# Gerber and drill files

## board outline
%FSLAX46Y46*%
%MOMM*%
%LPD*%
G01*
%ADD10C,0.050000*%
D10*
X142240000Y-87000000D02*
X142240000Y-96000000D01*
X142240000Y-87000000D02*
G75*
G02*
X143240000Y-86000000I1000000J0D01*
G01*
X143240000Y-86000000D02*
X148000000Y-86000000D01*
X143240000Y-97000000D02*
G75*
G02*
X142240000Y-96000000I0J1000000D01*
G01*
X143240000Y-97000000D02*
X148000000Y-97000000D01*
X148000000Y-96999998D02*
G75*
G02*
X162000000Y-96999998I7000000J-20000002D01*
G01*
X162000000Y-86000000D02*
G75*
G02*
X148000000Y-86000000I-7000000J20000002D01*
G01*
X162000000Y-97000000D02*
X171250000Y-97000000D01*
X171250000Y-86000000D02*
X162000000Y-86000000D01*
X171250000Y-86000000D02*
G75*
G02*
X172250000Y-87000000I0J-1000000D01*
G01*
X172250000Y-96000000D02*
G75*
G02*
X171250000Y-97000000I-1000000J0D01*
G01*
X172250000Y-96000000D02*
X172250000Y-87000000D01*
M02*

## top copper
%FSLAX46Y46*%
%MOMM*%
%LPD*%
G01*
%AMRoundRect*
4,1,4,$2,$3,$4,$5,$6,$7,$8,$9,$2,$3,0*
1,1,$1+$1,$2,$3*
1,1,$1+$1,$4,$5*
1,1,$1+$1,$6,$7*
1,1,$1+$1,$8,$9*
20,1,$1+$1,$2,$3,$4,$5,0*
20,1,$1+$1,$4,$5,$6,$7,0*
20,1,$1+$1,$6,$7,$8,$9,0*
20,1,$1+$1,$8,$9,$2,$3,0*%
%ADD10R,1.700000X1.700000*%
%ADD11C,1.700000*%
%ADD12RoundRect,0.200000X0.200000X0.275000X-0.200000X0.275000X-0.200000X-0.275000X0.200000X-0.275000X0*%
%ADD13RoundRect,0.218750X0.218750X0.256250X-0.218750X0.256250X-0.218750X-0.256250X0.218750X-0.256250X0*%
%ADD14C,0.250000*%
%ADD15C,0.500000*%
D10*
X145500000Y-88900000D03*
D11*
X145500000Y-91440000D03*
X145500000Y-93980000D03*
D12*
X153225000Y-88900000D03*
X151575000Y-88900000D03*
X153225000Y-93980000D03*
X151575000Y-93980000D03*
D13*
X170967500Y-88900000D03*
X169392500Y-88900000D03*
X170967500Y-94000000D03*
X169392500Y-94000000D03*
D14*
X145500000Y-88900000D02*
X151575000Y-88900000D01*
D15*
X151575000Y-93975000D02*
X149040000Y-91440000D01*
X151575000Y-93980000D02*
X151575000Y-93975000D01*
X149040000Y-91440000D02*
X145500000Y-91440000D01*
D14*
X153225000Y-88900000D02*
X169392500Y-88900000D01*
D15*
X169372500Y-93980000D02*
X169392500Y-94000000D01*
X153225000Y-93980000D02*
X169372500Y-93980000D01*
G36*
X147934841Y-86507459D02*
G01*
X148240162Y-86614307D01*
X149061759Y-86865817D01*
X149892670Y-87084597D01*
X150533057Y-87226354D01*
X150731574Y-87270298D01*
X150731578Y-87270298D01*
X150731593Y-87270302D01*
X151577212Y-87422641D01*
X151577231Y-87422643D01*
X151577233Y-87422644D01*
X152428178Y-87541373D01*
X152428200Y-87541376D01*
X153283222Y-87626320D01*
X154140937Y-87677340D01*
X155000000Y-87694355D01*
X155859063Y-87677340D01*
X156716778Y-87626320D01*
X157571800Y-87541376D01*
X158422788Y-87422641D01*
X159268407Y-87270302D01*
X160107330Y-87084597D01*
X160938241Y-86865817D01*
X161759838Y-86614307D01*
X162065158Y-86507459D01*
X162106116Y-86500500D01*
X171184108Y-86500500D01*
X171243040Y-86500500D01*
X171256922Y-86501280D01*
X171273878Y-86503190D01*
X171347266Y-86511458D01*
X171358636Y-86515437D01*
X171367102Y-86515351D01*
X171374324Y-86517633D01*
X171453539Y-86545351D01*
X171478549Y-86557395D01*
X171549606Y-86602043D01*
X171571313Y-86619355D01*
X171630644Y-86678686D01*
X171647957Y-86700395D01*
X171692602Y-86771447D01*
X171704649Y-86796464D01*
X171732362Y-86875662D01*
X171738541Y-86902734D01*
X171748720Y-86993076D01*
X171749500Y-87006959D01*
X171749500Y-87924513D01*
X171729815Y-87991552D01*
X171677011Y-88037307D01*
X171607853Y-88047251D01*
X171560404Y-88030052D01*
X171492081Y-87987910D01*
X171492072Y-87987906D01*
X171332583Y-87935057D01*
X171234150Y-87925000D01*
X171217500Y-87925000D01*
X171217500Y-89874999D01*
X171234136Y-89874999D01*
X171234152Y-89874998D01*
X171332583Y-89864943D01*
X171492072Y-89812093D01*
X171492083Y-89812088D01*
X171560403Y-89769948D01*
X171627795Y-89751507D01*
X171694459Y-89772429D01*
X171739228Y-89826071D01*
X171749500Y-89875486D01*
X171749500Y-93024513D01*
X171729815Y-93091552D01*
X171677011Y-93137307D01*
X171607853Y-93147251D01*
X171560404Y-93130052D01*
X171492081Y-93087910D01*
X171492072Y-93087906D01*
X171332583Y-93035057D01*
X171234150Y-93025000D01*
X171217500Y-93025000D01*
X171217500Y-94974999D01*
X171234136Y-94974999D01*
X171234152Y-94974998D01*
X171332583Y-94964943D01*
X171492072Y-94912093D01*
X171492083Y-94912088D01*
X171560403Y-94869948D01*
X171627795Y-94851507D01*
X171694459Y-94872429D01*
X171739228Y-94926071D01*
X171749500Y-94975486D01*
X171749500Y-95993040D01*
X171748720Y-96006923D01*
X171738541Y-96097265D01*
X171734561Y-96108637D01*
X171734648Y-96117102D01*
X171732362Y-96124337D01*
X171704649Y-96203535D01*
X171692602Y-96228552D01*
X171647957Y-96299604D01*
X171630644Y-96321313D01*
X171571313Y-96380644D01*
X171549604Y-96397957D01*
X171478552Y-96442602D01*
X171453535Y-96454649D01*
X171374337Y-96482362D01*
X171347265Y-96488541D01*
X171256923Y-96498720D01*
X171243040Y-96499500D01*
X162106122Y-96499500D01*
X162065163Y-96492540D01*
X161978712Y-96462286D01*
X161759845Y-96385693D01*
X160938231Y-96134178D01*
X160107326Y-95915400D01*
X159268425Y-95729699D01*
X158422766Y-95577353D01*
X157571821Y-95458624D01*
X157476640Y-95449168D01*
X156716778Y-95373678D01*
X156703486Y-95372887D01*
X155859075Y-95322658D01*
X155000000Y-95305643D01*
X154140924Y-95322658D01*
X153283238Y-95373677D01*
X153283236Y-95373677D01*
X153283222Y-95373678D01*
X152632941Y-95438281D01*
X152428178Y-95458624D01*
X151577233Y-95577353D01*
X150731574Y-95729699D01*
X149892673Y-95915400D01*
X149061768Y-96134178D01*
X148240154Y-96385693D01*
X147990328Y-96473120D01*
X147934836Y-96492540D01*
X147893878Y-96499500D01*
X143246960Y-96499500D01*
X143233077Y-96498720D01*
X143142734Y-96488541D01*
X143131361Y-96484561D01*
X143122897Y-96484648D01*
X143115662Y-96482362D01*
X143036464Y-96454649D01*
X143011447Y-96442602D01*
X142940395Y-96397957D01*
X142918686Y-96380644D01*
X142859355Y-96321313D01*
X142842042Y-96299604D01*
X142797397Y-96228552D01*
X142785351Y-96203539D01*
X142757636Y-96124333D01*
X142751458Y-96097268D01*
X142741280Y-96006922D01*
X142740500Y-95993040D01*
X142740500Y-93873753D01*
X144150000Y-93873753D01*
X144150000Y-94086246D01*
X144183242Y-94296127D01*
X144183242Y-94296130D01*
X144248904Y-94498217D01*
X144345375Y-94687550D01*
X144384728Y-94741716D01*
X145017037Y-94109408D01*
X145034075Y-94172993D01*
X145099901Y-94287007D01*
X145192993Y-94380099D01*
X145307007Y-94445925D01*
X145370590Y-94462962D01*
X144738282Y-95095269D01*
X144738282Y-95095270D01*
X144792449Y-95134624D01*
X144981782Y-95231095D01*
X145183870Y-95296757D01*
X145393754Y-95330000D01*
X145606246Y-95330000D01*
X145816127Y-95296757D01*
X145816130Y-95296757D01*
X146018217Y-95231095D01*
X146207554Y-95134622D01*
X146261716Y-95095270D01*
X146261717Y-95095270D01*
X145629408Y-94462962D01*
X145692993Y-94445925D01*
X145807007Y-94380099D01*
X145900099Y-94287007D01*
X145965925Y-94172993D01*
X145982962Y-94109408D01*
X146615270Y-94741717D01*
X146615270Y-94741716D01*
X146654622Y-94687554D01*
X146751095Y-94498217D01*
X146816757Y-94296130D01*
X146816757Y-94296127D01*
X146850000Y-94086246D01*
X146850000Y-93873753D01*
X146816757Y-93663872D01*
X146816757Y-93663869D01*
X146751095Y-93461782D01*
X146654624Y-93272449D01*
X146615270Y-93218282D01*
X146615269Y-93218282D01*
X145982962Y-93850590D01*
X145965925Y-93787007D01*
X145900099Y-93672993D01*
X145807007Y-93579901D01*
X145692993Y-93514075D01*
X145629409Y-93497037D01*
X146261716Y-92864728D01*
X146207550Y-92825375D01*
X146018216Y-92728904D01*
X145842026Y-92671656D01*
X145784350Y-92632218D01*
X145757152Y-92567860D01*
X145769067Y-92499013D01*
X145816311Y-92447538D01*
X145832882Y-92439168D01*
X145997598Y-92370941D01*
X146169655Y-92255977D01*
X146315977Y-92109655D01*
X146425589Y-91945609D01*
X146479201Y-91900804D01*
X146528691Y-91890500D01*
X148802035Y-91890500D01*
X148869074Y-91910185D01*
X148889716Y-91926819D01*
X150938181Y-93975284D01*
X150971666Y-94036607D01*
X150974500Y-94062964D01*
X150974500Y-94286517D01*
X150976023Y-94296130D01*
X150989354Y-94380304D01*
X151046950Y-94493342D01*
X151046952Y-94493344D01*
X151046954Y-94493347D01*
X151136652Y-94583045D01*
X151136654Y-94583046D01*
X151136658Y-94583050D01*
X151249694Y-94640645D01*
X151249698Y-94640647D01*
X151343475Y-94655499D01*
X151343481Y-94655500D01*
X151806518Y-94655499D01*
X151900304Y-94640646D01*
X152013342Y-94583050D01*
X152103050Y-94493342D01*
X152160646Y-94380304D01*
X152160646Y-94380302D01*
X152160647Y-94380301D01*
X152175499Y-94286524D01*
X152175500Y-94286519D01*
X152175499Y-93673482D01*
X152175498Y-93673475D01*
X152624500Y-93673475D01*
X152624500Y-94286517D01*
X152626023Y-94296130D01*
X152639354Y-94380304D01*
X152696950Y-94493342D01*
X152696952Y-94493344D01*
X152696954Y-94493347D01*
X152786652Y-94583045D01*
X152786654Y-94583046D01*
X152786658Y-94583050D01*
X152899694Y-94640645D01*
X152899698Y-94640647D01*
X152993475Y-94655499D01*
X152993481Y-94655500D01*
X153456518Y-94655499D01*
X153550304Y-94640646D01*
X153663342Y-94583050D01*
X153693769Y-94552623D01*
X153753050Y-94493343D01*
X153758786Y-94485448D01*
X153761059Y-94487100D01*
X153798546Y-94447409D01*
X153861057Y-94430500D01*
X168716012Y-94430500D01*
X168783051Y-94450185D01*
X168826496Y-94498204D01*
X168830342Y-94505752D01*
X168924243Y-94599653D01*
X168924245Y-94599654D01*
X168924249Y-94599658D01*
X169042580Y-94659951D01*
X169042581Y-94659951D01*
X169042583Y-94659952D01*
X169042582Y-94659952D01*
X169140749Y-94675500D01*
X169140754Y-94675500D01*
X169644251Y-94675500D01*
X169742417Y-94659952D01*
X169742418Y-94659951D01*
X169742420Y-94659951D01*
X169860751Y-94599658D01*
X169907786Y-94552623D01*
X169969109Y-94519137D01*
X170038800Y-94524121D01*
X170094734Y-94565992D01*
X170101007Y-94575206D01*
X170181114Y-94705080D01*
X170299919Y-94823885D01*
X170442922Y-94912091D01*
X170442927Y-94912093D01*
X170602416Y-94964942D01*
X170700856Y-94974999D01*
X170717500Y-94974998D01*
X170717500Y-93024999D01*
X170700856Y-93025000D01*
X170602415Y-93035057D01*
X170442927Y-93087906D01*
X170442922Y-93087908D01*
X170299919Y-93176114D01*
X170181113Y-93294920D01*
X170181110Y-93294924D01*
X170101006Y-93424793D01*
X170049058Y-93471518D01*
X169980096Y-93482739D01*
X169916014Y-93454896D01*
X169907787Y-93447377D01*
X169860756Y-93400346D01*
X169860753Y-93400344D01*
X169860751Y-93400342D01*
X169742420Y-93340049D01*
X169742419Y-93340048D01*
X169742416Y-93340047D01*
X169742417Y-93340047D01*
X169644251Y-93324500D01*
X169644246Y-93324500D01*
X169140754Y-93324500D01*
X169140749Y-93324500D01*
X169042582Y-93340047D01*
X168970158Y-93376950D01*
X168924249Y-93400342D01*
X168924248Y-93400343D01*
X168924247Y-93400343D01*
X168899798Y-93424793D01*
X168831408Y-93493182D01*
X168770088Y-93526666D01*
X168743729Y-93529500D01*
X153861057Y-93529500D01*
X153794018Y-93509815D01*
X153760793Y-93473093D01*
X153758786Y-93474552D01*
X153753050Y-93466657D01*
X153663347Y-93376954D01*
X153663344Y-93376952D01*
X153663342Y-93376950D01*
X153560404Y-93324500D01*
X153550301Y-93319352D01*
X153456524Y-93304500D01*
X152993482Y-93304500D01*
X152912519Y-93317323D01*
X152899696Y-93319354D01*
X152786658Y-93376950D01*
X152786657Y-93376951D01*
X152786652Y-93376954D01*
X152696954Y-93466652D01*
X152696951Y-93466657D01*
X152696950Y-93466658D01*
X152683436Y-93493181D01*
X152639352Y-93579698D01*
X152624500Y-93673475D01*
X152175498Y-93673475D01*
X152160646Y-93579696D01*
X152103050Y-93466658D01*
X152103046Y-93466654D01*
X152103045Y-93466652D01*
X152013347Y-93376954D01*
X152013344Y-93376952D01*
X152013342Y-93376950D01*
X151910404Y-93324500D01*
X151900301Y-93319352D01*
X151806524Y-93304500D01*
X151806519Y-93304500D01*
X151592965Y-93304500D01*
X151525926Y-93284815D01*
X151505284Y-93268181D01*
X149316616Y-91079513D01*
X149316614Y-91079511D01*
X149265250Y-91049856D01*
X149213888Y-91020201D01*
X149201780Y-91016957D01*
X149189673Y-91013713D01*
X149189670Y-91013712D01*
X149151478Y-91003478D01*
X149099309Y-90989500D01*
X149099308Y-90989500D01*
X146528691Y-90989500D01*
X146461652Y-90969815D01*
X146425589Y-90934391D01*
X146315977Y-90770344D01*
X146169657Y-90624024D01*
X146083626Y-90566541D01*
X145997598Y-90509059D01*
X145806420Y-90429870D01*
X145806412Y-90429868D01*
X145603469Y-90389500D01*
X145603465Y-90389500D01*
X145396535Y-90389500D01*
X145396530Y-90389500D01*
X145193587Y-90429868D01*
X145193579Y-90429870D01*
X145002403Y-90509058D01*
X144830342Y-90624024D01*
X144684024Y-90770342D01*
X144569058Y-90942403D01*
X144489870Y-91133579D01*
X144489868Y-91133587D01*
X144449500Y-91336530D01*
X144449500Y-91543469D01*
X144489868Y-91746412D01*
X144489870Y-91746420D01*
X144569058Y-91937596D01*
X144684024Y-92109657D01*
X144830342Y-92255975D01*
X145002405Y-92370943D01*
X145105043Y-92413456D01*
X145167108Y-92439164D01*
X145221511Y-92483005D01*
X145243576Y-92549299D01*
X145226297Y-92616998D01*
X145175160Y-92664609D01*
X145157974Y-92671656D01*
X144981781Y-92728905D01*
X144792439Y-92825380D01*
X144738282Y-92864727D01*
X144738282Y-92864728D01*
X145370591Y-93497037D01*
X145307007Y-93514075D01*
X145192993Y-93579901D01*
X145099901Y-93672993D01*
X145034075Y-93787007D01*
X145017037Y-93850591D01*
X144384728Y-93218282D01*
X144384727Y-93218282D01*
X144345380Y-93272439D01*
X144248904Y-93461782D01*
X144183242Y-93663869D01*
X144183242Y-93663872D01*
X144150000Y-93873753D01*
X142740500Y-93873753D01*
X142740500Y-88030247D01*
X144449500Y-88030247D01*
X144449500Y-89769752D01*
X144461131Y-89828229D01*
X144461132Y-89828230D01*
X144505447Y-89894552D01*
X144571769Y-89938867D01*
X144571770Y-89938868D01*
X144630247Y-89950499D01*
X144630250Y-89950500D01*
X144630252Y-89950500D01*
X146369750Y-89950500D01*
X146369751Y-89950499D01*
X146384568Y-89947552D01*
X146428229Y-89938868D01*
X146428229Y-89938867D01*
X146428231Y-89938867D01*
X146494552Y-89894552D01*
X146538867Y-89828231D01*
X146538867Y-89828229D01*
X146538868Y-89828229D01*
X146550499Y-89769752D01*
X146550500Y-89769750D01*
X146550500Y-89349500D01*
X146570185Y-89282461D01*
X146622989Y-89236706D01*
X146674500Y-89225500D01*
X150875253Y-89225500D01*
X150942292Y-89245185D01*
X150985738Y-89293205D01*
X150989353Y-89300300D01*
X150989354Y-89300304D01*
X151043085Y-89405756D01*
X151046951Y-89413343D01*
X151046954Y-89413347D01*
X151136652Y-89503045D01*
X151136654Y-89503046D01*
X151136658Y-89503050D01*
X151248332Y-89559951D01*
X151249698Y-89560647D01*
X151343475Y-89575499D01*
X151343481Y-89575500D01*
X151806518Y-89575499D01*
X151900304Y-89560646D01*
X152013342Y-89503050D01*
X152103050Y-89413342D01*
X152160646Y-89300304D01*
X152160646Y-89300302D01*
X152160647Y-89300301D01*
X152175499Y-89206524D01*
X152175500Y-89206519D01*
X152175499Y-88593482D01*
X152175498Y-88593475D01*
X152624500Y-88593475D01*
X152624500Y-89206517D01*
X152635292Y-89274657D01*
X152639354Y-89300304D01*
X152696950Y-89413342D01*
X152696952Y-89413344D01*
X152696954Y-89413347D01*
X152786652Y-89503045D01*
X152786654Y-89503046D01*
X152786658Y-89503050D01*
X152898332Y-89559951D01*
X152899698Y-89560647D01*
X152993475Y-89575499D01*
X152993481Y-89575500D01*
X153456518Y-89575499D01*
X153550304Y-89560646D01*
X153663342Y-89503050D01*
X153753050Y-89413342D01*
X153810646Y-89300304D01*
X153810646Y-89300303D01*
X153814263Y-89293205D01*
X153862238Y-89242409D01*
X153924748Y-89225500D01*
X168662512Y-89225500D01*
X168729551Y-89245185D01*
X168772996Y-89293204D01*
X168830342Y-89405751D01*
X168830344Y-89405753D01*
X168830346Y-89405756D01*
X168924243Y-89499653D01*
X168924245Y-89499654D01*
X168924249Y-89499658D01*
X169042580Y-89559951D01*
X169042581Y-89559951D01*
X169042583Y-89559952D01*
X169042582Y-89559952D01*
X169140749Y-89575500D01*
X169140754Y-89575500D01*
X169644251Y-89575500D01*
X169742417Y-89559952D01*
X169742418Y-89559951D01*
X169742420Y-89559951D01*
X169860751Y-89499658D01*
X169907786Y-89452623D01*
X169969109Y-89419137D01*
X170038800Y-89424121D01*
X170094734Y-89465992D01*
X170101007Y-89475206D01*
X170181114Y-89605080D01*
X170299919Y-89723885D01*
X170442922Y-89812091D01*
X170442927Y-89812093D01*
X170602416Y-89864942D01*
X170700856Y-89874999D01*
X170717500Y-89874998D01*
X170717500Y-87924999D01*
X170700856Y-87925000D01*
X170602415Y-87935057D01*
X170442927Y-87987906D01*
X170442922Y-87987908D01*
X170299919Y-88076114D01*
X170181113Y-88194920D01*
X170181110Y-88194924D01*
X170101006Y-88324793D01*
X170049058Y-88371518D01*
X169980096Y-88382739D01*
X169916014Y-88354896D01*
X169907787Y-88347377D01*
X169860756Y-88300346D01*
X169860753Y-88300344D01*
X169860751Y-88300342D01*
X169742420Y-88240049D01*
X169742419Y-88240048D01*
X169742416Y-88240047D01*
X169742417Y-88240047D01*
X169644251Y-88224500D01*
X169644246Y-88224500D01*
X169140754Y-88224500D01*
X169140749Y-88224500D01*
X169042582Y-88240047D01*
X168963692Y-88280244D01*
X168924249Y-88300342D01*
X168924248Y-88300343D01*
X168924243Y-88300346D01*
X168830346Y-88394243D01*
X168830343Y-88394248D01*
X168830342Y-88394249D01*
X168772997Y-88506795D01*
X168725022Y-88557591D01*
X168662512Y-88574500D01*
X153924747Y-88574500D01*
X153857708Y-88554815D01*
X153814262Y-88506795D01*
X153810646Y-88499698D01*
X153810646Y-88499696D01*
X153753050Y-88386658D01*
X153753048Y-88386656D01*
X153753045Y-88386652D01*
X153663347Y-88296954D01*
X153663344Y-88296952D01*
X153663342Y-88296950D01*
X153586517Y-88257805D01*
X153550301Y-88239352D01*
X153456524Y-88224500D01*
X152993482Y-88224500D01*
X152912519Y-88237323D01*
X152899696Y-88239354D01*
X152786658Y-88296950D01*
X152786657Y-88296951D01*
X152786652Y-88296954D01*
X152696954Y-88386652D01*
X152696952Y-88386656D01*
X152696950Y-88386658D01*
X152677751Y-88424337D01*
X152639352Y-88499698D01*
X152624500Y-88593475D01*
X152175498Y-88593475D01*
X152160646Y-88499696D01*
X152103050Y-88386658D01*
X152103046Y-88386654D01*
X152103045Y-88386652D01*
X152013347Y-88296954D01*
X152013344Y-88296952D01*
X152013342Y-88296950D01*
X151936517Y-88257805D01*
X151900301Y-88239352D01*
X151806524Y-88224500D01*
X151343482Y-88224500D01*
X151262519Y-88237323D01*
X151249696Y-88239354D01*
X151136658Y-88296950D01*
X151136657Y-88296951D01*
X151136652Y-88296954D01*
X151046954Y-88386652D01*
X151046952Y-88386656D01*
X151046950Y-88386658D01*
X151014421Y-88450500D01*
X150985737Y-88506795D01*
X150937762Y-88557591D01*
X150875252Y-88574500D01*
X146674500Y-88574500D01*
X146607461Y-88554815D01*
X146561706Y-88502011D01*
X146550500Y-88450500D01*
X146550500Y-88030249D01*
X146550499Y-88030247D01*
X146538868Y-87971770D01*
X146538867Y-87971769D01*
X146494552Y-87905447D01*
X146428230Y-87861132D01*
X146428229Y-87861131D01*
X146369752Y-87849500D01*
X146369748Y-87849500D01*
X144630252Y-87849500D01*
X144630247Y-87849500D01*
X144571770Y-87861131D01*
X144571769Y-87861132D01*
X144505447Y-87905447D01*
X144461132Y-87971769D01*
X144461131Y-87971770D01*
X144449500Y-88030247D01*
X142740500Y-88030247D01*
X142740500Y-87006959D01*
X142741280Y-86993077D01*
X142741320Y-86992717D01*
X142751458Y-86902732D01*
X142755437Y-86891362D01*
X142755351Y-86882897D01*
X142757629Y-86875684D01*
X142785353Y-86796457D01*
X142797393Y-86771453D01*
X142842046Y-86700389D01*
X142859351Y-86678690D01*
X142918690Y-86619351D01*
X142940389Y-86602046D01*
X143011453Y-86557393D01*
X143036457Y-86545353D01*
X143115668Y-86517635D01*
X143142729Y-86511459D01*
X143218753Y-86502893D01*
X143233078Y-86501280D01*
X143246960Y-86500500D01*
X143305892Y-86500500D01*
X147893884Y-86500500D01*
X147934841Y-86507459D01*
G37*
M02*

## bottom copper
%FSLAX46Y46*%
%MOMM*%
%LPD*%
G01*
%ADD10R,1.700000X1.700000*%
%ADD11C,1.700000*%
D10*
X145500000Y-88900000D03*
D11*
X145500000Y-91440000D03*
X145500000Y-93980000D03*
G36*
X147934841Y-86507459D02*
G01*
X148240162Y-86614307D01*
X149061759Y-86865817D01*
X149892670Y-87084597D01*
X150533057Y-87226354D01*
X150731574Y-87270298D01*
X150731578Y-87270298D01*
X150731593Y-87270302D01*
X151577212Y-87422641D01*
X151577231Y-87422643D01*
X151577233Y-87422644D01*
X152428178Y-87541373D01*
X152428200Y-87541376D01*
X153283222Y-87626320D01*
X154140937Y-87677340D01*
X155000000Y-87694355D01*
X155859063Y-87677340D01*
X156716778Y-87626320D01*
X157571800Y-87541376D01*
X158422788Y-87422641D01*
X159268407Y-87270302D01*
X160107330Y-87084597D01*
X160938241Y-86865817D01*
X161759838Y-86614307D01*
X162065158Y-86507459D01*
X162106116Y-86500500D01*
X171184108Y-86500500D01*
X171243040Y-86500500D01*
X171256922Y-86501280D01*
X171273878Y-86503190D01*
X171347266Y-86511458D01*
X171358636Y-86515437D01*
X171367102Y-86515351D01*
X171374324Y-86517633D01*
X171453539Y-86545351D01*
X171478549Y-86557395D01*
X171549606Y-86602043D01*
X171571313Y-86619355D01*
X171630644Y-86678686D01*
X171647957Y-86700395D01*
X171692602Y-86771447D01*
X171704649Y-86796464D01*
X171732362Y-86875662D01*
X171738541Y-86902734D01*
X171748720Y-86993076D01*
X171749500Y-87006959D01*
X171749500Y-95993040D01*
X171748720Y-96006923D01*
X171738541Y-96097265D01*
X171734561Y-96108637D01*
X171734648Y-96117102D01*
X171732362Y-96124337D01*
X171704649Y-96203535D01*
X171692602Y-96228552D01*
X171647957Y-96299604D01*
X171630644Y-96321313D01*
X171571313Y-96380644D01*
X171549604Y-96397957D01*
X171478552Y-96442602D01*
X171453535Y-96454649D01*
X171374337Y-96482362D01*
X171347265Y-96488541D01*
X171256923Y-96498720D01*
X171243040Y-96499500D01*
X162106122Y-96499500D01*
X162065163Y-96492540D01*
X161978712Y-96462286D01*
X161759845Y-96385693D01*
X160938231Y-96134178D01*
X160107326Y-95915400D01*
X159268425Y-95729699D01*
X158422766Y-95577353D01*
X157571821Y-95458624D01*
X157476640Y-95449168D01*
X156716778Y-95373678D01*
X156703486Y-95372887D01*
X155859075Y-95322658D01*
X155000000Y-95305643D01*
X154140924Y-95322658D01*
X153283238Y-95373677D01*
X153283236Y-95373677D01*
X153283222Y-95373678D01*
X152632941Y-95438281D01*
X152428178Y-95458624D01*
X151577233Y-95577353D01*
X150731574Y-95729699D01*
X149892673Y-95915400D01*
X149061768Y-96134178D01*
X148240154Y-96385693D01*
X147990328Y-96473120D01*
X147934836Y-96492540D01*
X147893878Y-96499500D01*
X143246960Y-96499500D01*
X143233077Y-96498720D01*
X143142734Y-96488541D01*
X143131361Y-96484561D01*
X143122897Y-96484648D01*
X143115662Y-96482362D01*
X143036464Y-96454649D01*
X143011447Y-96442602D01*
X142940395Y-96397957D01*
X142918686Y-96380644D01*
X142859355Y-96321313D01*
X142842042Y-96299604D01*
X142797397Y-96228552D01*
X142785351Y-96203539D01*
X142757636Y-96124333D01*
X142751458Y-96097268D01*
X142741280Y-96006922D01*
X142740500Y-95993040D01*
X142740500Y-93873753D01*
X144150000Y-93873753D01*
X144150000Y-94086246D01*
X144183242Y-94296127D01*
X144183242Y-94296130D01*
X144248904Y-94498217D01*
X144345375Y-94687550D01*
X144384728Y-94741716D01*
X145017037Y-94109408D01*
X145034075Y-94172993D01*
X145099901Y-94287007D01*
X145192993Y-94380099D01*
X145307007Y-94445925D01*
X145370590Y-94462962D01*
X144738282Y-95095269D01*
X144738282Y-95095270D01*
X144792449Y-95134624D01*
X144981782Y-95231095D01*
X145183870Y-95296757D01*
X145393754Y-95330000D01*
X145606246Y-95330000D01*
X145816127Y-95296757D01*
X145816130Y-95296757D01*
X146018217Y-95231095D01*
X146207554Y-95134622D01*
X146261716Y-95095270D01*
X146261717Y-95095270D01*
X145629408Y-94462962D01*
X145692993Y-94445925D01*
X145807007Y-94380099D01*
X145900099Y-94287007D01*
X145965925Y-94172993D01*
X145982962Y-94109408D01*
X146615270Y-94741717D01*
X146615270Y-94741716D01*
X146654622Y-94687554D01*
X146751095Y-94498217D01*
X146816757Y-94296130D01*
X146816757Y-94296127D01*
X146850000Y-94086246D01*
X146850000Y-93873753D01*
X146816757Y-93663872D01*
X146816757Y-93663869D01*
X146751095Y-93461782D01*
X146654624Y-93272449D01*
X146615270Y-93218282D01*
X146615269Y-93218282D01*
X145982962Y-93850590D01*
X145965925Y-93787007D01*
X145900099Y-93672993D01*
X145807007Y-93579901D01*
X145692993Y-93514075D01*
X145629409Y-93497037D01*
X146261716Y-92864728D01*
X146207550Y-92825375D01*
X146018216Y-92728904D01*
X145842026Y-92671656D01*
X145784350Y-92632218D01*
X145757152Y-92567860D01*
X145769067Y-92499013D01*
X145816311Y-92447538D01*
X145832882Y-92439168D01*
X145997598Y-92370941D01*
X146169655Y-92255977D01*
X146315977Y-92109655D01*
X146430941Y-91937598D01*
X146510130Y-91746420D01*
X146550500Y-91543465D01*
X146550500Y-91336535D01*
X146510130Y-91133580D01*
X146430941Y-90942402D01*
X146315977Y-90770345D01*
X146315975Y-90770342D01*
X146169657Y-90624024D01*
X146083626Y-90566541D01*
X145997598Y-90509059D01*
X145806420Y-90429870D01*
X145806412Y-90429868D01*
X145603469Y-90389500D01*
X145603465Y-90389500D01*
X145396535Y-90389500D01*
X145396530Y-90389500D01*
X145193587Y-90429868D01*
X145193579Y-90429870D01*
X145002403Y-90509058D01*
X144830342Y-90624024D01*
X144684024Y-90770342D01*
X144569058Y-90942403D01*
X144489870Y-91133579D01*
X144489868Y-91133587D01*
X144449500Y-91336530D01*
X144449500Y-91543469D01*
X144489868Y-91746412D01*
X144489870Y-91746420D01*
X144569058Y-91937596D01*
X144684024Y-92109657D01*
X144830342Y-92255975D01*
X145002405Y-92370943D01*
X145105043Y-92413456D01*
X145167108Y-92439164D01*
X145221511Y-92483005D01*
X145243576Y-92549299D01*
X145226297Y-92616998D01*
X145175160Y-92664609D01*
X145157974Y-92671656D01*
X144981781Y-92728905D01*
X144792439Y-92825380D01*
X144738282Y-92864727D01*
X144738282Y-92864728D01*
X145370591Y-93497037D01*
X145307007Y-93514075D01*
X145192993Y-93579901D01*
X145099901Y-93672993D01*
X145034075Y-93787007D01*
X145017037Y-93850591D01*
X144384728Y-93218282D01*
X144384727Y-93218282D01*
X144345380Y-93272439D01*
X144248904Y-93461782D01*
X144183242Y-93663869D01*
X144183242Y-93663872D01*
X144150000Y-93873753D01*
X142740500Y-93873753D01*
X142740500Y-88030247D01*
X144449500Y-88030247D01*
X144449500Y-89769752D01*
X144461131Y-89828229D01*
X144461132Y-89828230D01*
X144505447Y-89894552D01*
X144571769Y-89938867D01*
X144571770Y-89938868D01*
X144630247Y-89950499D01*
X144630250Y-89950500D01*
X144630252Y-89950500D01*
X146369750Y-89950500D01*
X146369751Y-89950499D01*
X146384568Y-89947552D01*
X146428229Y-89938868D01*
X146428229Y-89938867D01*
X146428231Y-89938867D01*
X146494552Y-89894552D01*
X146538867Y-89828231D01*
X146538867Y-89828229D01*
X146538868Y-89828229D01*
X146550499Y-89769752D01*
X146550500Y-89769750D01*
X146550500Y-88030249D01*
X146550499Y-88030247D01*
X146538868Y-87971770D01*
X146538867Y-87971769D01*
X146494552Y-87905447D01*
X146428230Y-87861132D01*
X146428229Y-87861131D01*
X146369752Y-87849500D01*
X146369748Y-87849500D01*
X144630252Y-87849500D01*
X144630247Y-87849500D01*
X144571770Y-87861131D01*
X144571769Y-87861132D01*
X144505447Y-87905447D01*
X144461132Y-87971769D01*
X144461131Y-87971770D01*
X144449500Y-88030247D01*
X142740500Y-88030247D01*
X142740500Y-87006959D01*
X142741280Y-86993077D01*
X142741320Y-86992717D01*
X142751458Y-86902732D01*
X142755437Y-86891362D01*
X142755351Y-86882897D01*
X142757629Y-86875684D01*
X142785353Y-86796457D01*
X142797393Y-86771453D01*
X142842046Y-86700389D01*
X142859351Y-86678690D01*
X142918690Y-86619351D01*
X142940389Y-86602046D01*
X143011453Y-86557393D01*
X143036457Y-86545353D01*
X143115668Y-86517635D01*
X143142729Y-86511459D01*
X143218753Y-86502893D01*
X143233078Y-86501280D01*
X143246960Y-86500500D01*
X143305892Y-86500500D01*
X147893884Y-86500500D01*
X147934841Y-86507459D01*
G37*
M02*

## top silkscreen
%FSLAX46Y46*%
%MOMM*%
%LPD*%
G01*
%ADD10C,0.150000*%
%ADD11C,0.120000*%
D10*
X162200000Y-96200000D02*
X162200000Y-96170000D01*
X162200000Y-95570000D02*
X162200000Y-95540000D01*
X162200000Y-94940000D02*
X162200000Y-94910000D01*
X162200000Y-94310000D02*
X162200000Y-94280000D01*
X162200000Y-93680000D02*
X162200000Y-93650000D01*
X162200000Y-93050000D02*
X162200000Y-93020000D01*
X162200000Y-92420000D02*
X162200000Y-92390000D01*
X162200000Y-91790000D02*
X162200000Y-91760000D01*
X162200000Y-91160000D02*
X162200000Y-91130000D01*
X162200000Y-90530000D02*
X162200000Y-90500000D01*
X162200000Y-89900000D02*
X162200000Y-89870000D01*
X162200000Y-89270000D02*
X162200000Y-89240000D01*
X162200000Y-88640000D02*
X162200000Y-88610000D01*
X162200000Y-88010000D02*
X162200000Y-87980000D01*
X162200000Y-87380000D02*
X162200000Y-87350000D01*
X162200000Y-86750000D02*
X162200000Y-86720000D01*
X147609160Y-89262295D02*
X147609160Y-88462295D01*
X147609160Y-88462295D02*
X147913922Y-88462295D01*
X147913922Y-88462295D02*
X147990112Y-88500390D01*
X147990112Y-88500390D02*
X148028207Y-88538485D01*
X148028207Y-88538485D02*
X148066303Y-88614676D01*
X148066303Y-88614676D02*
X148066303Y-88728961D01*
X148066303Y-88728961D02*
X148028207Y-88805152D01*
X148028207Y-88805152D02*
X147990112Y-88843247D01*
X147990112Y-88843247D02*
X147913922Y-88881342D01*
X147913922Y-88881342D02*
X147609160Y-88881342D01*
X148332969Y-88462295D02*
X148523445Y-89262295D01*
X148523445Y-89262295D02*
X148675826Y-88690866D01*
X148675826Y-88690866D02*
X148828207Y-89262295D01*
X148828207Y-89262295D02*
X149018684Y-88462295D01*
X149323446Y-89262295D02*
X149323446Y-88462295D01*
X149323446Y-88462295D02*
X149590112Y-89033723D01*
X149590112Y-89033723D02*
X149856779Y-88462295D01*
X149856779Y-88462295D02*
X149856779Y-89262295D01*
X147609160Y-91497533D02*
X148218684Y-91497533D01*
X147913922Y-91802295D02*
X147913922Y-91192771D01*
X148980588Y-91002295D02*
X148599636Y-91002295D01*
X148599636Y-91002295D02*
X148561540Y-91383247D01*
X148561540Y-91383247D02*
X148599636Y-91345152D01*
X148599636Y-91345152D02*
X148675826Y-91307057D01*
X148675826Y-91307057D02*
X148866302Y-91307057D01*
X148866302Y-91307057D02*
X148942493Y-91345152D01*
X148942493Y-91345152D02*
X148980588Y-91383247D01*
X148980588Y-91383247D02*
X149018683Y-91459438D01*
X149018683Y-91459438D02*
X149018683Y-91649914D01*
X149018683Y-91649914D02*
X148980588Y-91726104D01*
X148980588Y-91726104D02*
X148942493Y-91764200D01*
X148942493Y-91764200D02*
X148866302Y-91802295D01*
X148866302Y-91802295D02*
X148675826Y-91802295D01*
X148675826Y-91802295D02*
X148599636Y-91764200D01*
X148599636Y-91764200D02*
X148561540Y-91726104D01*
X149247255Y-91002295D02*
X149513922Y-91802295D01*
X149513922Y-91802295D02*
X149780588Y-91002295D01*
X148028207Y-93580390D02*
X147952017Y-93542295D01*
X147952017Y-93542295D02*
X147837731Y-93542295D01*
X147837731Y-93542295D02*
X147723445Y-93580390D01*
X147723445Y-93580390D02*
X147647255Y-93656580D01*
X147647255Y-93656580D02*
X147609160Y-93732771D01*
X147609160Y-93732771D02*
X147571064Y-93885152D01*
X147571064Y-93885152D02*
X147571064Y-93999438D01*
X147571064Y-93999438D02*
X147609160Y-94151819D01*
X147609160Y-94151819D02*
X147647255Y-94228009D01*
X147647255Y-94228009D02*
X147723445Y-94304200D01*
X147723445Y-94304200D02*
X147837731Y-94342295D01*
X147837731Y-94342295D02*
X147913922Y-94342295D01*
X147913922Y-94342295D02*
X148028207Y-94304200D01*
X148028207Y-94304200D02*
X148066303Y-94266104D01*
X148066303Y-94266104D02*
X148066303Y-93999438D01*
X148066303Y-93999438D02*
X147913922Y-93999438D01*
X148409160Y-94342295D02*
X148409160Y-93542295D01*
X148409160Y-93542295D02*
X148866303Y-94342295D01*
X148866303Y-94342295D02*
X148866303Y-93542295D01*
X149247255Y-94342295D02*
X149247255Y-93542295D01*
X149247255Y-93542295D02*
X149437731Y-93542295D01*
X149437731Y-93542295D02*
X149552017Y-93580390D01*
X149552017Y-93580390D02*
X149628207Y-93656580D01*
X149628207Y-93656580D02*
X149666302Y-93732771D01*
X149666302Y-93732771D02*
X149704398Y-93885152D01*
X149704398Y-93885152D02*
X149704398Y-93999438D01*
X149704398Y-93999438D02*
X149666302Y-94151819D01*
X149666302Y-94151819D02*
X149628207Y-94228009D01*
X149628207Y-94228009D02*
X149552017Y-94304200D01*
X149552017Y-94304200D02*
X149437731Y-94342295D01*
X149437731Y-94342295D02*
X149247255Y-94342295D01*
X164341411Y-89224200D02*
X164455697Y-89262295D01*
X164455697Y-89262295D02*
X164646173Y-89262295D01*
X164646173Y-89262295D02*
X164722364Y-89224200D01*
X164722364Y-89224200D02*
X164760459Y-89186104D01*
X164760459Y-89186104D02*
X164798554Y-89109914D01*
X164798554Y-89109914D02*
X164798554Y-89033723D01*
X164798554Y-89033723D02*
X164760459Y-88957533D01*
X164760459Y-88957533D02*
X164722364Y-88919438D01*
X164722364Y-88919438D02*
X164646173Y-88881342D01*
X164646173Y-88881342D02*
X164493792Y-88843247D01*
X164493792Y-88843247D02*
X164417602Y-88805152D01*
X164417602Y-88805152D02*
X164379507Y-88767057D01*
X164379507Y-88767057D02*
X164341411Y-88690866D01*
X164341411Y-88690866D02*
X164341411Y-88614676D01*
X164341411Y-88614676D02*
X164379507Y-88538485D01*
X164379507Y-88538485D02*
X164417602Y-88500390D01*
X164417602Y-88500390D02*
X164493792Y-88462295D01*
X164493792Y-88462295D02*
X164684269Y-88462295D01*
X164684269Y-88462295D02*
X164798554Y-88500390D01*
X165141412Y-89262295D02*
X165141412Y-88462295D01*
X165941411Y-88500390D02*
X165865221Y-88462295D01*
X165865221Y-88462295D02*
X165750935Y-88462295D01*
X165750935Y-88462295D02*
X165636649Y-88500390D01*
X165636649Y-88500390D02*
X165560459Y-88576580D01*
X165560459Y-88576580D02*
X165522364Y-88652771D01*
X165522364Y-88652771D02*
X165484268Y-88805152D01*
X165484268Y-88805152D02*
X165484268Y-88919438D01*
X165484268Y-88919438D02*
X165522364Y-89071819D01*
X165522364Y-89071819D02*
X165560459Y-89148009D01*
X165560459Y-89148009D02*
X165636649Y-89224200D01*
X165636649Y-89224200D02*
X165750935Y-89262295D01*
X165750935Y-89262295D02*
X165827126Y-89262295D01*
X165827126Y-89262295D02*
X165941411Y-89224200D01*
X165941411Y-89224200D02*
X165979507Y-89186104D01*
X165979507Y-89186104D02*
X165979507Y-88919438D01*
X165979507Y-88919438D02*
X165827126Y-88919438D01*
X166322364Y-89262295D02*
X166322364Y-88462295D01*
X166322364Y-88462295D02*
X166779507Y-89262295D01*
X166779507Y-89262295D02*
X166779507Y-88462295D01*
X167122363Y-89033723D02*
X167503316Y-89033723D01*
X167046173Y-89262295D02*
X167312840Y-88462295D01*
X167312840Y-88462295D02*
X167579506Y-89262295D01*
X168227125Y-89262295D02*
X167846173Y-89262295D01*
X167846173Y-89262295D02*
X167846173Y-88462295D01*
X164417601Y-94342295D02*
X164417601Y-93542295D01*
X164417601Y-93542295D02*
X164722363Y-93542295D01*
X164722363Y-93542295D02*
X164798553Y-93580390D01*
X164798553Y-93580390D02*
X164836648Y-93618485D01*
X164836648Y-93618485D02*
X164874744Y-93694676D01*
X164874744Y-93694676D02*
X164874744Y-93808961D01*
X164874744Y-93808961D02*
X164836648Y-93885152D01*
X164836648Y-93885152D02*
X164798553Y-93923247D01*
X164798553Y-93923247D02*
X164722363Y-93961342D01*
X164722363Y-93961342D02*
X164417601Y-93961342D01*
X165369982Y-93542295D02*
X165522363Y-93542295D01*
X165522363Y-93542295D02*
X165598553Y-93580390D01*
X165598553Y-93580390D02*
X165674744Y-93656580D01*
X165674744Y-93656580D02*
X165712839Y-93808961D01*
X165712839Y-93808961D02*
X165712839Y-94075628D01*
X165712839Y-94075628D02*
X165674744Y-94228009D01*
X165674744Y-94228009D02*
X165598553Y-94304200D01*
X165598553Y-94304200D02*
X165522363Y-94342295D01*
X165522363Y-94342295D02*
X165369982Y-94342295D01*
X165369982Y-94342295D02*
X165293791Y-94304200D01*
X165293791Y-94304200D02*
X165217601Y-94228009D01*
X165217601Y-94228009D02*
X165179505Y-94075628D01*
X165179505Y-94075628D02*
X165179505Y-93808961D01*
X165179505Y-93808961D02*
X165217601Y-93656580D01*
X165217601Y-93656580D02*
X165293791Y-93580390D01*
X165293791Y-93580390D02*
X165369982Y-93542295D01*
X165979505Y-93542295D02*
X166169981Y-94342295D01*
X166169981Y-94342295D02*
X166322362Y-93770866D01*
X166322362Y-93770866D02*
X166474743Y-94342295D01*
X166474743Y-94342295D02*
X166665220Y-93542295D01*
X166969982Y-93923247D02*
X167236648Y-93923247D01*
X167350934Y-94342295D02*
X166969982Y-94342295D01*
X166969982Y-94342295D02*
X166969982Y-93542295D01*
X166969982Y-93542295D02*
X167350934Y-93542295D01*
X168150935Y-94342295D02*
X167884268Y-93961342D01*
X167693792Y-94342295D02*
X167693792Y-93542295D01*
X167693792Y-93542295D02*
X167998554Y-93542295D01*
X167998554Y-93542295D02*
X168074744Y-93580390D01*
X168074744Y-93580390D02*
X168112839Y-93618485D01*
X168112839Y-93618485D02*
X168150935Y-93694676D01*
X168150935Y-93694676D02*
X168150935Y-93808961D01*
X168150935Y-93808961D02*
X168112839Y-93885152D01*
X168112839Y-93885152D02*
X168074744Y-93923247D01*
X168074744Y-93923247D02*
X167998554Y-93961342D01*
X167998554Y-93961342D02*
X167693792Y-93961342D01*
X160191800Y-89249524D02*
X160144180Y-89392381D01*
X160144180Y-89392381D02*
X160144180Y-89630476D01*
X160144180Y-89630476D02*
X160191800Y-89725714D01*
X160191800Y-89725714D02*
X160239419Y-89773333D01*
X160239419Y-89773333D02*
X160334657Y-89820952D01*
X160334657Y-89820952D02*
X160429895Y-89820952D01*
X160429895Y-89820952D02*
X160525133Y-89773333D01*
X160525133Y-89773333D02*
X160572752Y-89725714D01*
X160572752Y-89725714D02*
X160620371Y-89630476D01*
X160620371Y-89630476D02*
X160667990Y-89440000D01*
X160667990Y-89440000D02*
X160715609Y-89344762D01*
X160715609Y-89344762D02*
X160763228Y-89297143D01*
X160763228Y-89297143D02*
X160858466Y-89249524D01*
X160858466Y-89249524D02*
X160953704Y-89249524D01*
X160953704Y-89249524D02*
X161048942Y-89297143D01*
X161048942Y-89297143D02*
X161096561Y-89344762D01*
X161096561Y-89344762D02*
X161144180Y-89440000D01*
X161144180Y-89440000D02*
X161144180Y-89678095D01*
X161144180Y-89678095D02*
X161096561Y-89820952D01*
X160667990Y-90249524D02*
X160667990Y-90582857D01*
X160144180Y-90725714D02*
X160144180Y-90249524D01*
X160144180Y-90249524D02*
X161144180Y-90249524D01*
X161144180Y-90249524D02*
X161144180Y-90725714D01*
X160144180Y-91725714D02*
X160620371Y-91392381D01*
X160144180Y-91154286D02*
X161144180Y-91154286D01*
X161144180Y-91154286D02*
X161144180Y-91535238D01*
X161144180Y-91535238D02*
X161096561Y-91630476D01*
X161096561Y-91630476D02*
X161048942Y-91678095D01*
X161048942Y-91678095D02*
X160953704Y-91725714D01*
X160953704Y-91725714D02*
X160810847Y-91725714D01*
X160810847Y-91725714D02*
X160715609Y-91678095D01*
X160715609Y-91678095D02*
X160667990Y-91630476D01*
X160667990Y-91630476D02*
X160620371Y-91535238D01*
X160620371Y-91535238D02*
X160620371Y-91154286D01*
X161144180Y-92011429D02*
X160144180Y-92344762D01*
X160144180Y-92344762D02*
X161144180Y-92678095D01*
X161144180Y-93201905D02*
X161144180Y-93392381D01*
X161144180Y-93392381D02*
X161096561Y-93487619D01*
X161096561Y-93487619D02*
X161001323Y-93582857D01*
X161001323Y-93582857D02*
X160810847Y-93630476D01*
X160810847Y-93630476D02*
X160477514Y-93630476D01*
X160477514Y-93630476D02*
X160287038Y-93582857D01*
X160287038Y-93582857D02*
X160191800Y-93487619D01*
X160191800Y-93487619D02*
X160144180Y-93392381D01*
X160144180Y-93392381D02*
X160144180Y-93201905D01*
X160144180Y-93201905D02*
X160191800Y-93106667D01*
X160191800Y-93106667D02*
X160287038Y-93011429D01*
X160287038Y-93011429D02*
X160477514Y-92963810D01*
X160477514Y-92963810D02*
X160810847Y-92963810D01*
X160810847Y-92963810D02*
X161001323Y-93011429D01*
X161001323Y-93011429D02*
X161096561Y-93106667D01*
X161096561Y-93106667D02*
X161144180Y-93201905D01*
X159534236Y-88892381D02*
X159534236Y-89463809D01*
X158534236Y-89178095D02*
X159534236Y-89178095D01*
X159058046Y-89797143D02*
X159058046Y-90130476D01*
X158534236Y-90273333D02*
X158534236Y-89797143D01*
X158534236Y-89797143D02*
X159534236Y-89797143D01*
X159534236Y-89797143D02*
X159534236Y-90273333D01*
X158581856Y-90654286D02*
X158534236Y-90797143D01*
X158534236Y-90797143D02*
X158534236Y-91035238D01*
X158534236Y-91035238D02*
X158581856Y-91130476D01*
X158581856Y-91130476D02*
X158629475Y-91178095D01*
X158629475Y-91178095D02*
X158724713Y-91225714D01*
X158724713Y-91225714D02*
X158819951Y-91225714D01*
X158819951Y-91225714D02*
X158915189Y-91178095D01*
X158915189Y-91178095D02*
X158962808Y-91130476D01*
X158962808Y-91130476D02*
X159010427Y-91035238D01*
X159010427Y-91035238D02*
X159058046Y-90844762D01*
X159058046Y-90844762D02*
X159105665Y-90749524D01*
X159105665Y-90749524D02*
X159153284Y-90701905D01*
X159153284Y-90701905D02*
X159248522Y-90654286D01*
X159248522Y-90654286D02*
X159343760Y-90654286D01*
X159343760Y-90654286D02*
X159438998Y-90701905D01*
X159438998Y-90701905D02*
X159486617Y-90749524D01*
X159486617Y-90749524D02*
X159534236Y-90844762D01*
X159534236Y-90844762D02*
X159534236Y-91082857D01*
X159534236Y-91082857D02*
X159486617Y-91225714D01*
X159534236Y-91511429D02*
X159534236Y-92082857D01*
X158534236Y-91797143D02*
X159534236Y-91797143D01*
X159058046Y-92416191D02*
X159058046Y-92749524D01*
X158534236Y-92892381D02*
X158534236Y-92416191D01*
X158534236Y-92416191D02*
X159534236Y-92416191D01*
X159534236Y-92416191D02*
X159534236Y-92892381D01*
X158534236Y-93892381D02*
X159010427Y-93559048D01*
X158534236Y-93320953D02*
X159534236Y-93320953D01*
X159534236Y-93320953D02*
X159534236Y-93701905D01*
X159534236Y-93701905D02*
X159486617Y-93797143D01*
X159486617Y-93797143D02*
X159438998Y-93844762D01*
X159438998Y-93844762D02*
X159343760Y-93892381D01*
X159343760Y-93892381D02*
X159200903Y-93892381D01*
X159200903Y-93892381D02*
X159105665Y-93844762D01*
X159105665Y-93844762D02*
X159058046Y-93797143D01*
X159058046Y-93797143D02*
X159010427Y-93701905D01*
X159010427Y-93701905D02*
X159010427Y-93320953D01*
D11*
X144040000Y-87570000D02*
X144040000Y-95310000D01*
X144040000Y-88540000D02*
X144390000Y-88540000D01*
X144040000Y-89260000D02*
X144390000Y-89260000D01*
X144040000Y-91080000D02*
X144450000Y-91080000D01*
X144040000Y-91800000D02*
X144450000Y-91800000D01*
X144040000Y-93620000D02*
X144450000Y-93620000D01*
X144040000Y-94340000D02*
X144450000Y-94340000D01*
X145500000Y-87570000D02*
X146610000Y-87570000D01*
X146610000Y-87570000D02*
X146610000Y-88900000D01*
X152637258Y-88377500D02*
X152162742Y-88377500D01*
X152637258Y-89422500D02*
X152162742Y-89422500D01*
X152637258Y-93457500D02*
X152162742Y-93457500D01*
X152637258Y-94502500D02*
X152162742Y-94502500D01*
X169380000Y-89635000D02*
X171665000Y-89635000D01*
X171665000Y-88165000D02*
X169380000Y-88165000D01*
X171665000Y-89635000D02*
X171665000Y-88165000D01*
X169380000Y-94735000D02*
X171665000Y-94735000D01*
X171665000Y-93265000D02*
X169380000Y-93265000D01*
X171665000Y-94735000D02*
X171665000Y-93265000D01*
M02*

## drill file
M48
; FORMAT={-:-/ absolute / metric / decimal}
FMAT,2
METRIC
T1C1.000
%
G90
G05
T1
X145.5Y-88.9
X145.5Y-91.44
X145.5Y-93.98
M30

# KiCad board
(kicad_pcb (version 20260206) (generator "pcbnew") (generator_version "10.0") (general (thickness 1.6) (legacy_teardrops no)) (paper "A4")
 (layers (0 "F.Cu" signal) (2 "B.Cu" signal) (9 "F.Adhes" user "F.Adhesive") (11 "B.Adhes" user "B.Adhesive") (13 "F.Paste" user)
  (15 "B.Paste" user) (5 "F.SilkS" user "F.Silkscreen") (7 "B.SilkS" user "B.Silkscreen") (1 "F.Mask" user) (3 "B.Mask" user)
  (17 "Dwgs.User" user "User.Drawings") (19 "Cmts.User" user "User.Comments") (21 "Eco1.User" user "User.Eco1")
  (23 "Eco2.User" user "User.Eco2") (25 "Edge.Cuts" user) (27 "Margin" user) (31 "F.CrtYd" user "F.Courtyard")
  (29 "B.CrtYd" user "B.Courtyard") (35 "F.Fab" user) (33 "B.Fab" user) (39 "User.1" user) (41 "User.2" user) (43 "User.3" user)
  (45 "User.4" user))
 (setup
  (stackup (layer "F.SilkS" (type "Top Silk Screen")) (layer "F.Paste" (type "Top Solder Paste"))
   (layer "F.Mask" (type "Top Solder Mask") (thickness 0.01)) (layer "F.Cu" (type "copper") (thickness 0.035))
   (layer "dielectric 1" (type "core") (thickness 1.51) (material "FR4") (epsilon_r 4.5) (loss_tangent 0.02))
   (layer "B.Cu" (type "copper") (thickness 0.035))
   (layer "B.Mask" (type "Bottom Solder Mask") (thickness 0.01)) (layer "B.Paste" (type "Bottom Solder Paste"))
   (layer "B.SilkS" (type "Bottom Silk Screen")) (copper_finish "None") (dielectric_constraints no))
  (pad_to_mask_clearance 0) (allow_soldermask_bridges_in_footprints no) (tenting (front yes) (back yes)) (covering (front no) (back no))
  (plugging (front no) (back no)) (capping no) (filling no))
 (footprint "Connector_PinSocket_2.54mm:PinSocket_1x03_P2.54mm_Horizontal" (layer "F.Cu") (at 145.5 88.9)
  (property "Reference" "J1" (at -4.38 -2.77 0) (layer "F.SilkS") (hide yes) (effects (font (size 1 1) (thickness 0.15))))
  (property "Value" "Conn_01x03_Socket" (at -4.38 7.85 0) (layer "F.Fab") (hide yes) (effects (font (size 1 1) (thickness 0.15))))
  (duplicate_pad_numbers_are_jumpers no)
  (fp_line (start -1.46 -1.33) (end -1.46 6.41) (stroke (width 0.12) (type solid)) (layer "F.SilkS"))
  (fp_line (start -1.46 -0.36) (end -1.11 -0.36) (stroke (width 0.12) (type solid)) (layer "F.SilkS"))
  (fp_line (start -1.46 0.36) (end -1.11 0.36) (stroke (width 0.12) (type solid)) (layer "F.SilkS"))
  (fp_line (start -1.46 2.18) (end -1.05 2.18) (stroke (width 0.12) (type solid)) (layer "F.SilkS"))
  (fp_line (start -1.46 2.9) (end -1.05 2.9) (stroke (width 0.12) (type solid)) (layer "F.SilkS"))
  (fp_line (start -1.46 4.72) (end -1.05 4.72) (stroke (width 0.12) (type solid)) (layer "F.SilkS"))
  (fp_line (start -1.46 5.44) (end -1.05 5.44) (stroke (width 0.12) (type solid)) (layer "F.SilkS"))
  (fp_line (start 0 -1.33) (end 1.11 -1.33) (stroke (width 0.12) (type solid)) (layer "F.SilkS"))
  (fp_line (start 1.11 -1.33) (end 1.11 0) (stroke (width 0.12) (type solid)) (layer "F.SilkS"))
  (pad "1" thru_hole rect (at 0 0) (size 1.7 1.7) (drill 1) (layers "*.Cu" "*.Mask") (remove_unused_layers no) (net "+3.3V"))
  (pad "2" thru_hole circle (at 0 2.54) (size 1.7 1.7) (drill 1) (layers "*.Cu" "*.Mask") (remove_unused_layers no) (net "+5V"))
  (pad "3" thru_hole circle (at 0 5.08) (size 1.7 1.7) (drill 1) (layers "*.Cu" "*.Mask") (remove_unused_layers no) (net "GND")))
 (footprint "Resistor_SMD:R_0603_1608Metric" (layer "F.Cu") (at 152.4 88.9 180)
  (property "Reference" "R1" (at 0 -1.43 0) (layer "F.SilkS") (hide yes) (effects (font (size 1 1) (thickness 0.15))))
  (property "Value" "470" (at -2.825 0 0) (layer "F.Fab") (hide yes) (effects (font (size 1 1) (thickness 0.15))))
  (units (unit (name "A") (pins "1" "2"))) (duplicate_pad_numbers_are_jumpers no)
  (fp_line (start -0.237258 0.5225) (end 0.237258 0.5225) (stroke (width 0.12) (type solid)) (layer "F.SilkS"))
  (fp_line (start -0.237258 -0.5225) (end 0.237258 -0.5225) (stroke (width 0.12) (type solid)) (layer "F.SilkS"))
  (pad "1" smd roundrect (at -0.825 0 180) (size 0.8 0.95) (layers "F.Cu" "F.Mask" "F.Paste") (roundrect_rratio 0.25) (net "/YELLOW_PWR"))
  (pad "2" smd roundrect (at 0.825 0 180) (size 0.8 0.95) (layers "F.Cu" "F.Mask" "F.Paste") (roundrect_rratio 0.25) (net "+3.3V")))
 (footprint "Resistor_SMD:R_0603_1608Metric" (layer "F.Cu") (at 152.4 93.98 180)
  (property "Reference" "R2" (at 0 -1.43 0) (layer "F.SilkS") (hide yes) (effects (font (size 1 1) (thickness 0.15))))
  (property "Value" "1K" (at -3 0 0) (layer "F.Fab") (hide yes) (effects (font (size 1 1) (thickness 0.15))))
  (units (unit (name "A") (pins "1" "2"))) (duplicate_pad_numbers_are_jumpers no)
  (fp_line (start -0.237258 0.5225) (end 0.237258 0.5225) (stroke (width 0.12) (type solid)) (layer "F.SilkS"))
  (fp_line (start -0.237258 -0.5225) (end 0.237258 -0.5225) (stroke (width 0.12) (type solid)) (layer "F.SilkS"))
  (pad "1" smd roundrect (at -0.825 0 180) (size 0.8 0.95) (layers "F.Cu" "F.Mask" "F.Paste") (roundrect_rratio 0.25) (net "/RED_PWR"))
  (pad "2" smd roundrect (at 0.825 0 180) (size 0.8 0.95) (layers "F.Cu" "F.Mask" "F.Paste") (roundrect_rratio 0.25) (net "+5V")))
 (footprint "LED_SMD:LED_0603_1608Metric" (layer "F.Cu") (at 170.18 88.9 180)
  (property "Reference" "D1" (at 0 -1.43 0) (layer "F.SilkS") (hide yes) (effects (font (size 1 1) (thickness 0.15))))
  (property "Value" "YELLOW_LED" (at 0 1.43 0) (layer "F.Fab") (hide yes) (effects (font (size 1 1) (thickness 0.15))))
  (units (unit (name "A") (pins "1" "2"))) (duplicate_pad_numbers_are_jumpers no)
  (fp_line (start 0.8 -0.735) (end -1.485 -0.735) (stroke (width 0.12) (type solid)) (layer "F.SilkS"))
  (fp_line (start -1.485 0.735) (end 0.8 0.735) (stroke (width 0.12) (type solid)) (layer "F.SilkS"))
  (fp_line (start -1.485 -0.735) (end -1.485 0.735) (stroke (width 0.12) (type solid)) (layer "F.SilkS"))
  (pad "1" smd roundrect (at -0.7875 0 180) (size 0.875 0.95) (layers "F.Cu" "F.Mask" "F.Paste") (roundrect_rratio 0.25) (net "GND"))
  (pad "2" smd roundrect (at 0.7875 0 180) (size 0.875 0.95) (layers "F.Cu" "F.Mask" "F.Paste") (roundrect_rratio 0.25) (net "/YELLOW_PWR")))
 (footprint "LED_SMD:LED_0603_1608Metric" (layer "F.Cu") (at 170.18 94 180)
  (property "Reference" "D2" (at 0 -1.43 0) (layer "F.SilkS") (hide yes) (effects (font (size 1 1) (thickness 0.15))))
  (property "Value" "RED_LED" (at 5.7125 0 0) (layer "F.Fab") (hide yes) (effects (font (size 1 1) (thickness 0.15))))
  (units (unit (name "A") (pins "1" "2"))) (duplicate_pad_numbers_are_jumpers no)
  (fp_line (start 0.8 -0.735) (end -1.485 -0.735) (stroke (width 0.12) (type solid)) (layer "F.SilkS"))
  (fp_line (start -1.485 0.735) (end 0.8 0.735) (stroke (width 0.12) (type solid)) (layer "F.SilkS"))
  (fp_line (start -1.485 -0.735) (end -1.485 0.735) (stroke (width 0.12) (type solid)) (layer "F.SilkS"))
  (pad "1" smd roundrect (at -0.7875 0 180) (size 0.875 0.95) (layers "F.Cu" "F.Mask" "F.Paste") (roundrect_rratio 0.25) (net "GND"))
  (pad "2" smd roundrect (at 0.7875 0 180) (size 0.875 0.95) (layers "F.Cu" "F.Mask" "F.Paste") (roundrect_rratio 0.25) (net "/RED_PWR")))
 (gr_line (start 162.2 96.2) (end 162.2 86.6) (stroke (width 0.15) (type dot)) (layer "F.SilkS"))
 (gr_line (start 142.24 87) (end 142.24 96) (stroke (width 0.05) (type default)) (layer "Edge.Cuts"))
 (gr_arc (start 142.24 87) (mid 142.532893 86.292893) (end 143.24 86) (stroke (width 0.05) (type default)) (layer "Edge.Cuts"))
 (gr_line (start 143.24 86) (end 148 86) (stroke (width 0.05) (type solid)) (layer "Edge.Cuts"))
 (gr_arc (start 143.24 97) (mid 142.532893 96.707107) (end 142.24 96) (stroke (width 0.05) (type default)) (layer "Edge.Cuts"))
 (gr_line (start 143.24 97) (end 148 97) (stroke (width 0.05) (type default)) (layer "Edge.Cuts"))
 (gr_arc (start 148 96.999998) (mid 155 95.810378) (end 162 96.999998) (stroke (width 0.05) (type default)) (layer "Edge.Cuts"))
 (gr_arc (start 162 86) (mid 155 87.18962) (end 148 86) (stroke (width 0.05) (type default)) (layer "Edge.Cuts"))
 (gr_line (start 162 97) (end 171.25 97) (stroke (width 0.05) (type default)) (layer "Edge.Cuts"))
 (gr_line (start 171.25 86) (end 162 86) (stroke (width 0.05) (type default)) (layer "Edge.Cuts"))
 (gr_arc (start 171.25 86) (mid 171.957107 86.292893) (end 172.25 87) (stroke (width 0.05) (type default)) (layer "Edge.Cuts"))
 (gr_arc (start 172.25 96) (mid 171.957107 96.707107) (end 171.25 97) (stroke (width 0.05) (type default)) (layer "Edge.Cuts"))
 (gr_line (start 172.25 96) (end 172.25 87) (stroke (width 0.05) (type default)) (layer "Edge.Cuts"))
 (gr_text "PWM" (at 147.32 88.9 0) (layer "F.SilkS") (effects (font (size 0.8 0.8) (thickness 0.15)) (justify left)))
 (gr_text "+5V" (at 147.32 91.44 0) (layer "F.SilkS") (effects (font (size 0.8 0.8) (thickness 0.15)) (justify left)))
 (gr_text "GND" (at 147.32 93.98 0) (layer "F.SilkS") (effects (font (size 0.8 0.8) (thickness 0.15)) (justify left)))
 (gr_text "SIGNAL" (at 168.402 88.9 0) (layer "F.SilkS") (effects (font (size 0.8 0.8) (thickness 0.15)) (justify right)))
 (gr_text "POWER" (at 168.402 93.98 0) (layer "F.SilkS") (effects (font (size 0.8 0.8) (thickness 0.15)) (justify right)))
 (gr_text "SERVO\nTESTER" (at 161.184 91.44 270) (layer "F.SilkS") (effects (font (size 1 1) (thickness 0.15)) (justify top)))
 (segment (start 145.5 88.9) (end 151.575 88.9) (width 0.25) (layer "F.Cu") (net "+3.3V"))
 (segment (start 151.575 93.975) (end 149.04 91.44) (width 0.5) (layer "F.Cu") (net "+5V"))
 (segment (start 151.575 93.98) (end 151.575 93.975) (width 0.5) (layer "F.Cu") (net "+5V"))
 (segment (start 149.04 91.44) (end 145.5 91.44) (width 0.5) (layer "F.Cu") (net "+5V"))
 (segment (start 153.225 88.9) (end 169.3925 88.9) (width 0.25) (layer "F.Cu") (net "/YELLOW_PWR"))
 (segment (start 169.3725 93.98) (end 169.3925 94) (width 0.5) (layer "F.Cu") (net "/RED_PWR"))
 (segment (start 153.225 93.98) (end 169.3725 93.98) (width 0.5) (layer "F.Cu") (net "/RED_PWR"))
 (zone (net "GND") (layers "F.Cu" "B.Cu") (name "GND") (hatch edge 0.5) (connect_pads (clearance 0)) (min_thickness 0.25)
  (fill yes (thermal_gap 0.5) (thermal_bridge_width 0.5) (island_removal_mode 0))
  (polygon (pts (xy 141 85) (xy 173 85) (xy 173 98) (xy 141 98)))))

